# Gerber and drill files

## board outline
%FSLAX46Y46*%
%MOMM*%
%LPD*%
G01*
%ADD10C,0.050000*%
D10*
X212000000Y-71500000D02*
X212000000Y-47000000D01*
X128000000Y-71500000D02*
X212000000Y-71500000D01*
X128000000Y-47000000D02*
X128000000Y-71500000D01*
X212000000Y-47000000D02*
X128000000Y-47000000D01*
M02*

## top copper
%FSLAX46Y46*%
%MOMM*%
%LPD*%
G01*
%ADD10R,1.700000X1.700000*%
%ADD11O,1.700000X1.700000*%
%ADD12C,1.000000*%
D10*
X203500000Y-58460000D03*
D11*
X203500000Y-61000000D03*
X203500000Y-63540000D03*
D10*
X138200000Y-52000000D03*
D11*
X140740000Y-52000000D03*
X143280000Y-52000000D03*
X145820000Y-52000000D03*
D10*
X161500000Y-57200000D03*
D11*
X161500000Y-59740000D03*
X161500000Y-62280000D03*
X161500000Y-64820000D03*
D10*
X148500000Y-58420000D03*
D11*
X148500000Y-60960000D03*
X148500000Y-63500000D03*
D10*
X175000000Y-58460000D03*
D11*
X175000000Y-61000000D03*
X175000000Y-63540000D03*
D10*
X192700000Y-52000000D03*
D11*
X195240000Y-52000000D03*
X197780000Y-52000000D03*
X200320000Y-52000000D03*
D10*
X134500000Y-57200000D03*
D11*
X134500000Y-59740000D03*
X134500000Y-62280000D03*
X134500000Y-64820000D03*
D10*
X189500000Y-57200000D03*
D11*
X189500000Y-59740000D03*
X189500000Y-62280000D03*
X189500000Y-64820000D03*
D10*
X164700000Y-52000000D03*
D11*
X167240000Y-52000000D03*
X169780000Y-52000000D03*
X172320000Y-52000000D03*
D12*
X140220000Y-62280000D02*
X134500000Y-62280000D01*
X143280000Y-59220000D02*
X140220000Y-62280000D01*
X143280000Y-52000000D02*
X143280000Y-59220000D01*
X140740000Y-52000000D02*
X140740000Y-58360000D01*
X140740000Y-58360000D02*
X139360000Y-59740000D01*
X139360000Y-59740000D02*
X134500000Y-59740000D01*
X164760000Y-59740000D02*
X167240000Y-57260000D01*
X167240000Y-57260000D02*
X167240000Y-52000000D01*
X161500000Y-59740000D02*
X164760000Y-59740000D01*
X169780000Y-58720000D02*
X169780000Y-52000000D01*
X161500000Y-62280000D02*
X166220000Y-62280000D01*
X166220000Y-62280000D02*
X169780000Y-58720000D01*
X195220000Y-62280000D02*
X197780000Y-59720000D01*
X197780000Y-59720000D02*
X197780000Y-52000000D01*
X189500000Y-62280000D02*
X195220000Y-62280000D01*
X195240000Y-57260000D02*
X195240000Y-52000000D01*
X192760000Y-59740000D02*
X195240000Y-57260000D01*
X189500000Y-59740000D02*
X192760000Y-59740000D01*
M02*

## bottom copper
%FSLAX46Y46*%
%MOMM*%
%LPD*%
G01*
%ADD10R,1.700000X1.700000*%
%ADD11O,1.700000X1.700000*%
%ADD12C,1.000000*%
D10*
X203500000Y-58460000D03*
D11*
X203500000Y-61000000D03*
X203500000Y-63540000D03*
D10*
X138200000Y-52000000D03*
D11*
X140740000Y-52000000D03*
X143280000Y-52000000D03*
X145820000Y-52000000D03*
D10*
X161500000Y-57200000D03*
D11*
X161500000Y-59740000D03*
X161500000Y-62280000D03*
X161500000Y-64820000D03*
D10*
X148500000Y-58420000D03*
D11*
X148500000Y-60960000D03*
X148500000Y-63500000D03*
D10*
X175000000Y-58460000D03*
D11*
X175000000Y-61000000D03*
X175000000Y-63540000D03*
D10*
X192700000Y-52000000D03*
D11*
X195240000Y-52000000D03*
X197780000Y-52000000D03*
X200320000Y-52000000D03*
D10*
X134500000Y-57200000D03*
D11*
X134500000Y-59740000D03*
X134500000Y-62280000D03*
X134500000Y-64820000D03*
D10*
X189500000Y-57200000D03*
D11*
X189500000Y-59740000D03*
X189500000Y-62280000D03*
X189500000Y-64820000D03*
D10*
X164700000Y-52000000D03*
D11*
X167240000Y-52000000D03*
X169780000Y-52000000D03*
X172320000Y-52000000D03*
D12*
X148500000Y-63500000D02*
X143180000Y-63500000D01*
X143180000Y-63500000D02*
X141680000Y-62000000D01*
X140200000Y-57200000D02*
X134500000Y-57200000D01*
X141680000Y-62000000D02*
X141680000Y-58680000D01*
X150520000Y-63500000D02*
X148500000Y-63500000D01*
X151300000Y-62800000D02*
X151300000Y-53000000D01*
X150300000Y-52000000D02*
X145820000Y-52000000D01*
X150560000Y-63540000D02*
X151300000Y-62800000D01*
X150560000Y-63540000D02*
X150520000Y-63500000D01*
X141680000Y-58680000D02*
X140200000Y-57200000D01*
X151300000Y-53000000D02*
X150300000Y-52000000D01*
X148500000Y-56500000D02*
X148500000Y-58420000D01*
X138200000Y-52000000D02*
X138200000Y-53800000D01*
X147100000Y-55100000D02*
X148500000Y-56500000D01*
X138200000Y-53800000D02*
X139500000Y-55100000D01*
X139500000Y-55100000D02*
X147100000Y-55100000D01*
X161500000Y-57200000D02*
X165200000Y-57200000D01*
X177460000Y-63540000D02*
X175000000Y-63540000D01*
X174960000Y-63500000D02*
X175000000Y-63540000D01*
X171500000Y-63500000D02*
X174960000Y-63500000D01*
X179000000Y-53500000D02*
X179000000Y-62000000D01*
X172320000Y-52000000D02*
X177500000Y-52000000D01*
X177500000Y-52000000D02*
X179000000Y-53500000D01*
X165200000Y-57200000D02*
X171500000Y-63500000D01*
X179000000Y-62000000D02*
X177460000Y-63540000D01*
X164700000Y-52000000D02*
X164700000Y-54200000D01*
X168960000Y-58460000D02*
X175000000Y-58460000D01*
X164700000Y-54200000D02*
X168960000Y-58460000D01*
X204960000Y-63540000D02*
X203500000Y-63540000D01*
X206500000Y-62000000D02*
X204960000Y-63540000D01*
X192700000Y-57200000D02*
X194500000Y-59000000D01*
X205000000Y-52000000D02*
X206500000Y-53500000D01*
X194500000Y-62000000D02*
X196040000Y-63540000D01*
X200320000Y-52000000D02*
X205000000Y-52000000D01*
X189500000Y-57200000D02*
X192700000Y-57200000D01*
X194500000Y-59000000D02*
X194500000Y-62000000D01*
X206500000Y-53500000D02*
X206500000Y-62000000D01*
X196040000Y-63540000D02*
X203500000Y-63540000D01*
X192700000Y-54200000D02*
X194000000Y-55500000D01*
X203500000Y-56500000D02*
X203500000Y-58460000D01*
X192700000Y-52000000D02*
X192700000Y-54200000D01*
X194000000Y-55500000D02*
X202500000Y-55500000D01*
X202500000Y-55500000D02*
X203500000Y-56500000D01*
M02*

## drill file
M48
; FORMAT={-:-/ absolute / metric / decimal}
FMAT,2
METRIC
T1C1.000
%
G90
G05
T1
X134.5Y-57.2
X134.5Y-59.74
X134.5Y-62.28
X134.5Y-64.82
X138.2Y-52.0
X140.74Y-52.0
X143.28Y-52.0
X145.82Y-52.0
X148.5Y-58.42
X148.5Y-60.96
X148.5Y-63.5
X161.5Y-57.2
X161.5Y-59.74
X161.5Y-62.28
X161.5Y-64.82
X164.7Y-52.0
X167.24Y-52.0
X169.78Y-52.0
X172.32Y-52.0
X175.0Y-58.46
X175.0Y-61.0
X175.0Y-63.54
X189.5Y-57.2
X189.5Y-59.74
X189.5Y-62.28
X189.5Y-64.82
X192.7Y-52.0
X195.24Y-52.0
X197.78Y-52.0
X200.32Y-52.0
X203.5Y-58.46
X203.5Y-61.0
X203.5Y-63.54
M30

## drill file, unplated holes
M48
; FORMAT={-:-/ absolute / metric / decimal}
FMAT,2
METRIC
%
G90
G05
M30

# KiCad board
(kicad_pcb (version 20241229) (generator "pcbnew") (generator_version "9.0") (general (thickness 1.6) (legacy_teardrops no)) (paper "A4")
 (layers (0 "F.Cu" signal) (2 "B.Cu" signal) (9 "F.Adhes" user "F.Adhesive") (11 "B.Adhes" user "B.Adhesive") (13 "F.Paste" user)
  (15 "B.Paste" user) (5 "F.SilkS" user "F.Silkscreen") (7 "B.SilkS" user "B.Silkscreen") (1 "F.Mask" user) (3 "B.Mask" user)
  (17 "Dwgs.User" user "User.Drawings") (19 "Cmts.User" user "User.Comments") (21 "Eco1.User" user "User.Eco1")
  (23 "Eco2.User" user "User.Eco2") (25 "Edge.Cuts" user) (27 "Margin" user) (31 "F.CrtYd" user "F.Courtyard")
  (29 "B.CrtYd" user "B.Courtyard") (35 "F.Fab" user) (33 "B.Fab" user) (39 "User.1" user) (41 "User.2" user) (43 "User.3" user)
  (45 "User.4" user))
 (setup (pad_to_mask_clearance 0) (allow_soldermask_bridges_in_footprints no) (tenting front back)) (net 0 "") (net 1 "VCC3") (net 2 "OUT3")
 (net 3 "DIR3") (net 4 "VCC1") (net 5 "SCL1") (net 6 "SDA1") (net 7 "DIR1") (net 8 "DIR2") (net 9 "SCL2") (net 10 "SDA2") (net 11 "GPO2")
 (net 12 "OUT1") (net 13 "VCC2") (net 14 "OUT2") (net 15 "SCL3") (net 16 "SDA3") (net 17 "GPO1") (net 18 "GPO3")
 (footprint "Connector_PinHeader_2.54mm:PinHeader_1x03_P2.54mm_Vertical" (layer "F.Cu") (at 203.5 58.46)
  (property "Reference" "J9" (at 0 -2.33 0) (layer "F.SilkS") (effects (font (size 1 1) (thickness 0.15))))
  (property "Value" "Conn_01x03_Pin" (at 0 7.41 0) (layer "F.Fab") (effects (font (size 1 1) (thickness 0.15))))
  (pad "1" thru_hole rect (at 0 0) (size 1.7 1.7) (drill 1) (layers "*.Cu" "*.Mask") (remove_unused_layers no) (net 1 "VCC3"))
  (pad "2" thru_hole oval (at 0 2.54) (size 1.7 1.7) (drill 1) (layers "*.Cu" "*.Mask") (remove_unused_layers no) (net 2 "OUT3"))
  (pad "3" thru_hole oval (at 0 5.08) (size 1.7 1.7) (drill 1) (layers "*.Cu" "*.Mask") (remove_unused_layers no) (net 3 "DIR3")))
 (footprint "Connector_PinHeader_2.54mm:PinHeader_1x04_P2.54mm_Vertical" (layer "F.Cu") (at 138.2 52 90)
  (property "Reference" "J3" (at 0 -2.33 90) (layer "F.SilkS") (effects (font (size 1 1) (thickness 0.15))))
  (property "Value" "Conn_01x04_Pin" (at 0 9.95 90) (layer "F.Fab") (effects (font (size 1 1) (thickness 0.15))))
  (pad "1" thru_hole rect (at 0 0 90) (size 1.7 1.7) (drill 1) (layers "*.Cu" "*.Mask") (remove_unused_layers no) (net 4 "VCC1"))
  (pad "2" thru_hole oval (at 0 2.54 90) (size 1.7 1.7) (drill 1) (layers "*.Cu" "*.Mask") (remove_unused_layers no) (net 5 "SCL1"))
  (pad "3" thru_hole oval (at 0 5.08 90) (size 1.7 1.7) (drill 1) (layers "*.Cu" "*.Mask") (remove_unused_layers no) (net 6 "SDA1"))
  (pad "4" thru_hole oval (at 0 7.62 90) (size 1.7 1.7) (drill 1) (layers "*.Cu" "*.Mask") (remove_unused_layers no) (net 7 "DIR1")))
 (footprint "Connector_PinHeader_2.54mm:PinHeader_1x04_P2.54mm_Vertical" (layer "F.Cu") (at 161.5 57.2)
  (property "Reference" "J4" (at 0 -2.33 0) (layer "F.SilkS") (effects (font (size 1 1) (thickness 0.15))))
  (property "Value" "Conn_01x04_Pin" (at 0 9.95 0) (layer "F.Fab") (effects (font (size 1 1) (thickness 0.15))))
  (pad "1" thru_hole rect (at 0 0) (size 1.7 1.7) (drill 1) (layers "*.Cu" "*.Mask") (remove_unused_layers no) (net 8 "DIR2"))
  (pad "2" thru_hole oval (at 0 2.54) (size 1.7 1.7) (drill 1) (layers "*.Cu" "*.Mask") (remove_unused_layers no) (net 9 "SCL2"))
  (pad "3" thru_hole oval (at 0 5.08) (size 1.7 1.7) (drill 1) (layers "*.Cu" "*.Mask") (remove_unused_layers no) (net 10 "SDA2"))
  (pad "4" thru_hole oval (at 0 7.62) (size 1.7 1.7) (drill 1) (layers "*.Cu" "*.Mask") (remove_unused_layers no) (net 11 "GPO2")))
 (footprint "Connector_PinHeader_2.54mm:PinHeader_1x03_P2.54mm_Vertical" (layer "F.Cu") (at 148.5 58.42)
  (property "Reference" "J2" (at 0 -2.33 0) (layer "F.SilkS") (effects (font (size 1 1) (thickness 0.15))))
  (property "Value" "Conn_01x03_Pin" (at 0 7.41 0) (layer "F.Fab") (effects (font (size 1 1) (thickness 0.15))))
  (pad "1" thru_hole rect (at 0 0) (size 1.7 1.7) (drill 1) (layers "*.Cu" "*.Mask") (remove_unused_layers no) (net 4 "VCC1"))
  (pad "2" thru_hole oval (at 0 2.54) (size 1.7 1.7) (drill 1) (layers "*.Cu" "*.Mask") (remove_unused_layers no) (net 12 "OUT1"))
  (pad "3" thru_hole oval (at 0 5.08) (size 1.7 1.7) (drill 1) (layers "*.Cu" "*.Mask") (remove_unused_layers no) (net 7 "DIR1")))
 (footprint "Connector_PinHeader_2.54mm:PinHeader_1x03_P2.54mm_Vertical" (layer "F.Cu") (at 175 58.46)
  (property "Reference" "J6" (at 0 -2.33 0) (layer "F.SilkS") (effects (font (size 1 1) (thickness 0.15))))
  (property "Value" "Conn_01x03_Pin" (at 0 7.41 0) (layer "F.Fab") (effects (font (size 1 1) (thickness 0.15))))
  (pad "1" thru_hole rect (at 0 0) (size 1.7 1.7) (drill 1) (layers "*.Cu" "*.Mask") (remove_unused_layers no) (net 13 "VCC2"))
  (pad "2" thru_hole oval (at 0 2.54) (size 1.7 1.7) (drill 1) (layers "*.Cu" "*.Mask") (remove_unused_layers no) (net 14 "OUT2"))
  (pad "3" thru_hole oval (at 0 5.08) (size 1.7 1.7) (drill 1) (layers "*.Cu" "*.Mask") (remove_unused_layers no) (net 8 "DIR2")))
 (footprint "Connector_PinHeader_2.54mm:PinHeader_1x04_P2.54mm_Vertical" (layer "F.Cu") (at 192.7 52 90)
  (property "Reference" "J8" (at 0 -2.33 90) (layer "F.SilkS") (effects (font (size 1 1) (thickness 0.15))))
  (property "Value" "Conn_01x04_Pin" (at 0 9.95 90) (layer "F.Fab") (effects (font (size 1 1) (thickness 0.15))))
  (pad "1" thru_hole rect (at 0 0 90) (size 1.7 1.7) (drill 1) (layers "*.Cu" "*.Mask") (remove_unused_layers no) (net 1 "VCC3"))
  (pad "2" thru_hole oval (at 0 2.54 90) (size 1.7 1.7) (drill 1) (layers "*.Cu" "*.Mask") (remove_unused_layers no) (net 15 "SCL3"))
  (pad "3" thru_hole oval (at 0 5.08 90) (size 1.7 1.7) (drill 1) (layers "*.Cu" "*.Mask") (remove_unused_layers no) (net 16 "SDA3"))
  (pad "4" thru_hole oval (at 0 7.62 90) (size 1.7 1.7) (drill 1) (layers "*.Cu" "*.Mask") (remove_unused_layers no) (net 3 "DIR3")))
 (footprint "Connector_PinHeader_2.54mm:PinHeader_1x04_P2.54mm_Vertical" (layer "F.Cu") (at 134.5 57.2)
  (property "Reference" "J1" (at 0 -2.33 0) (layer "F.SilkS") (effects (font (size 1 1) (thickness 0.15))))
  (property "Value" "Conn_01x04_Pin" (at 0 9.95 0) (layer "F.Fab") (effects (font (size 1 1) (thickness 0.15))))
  (pad "1" thru_hole rect (at 0 0) (size 1.7 1.7) (drill 1) (layers "*.Cu" "*.Mask") (remove_unused_layers no) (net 7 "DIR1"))
  (pad "2" thru_hole oval (at 0 2.54) (size 1.7 1.7) (drill 1) (layers "*.Cu" "*.Mask") (remove_unused_layers no) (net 5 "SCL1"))
  (pad "3" thru_hole oval (at 0 5.08) (size 1.7 1.7) (drill 1) (layers "*.Cu" "*.Mask") (remove_unused_layers no) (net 6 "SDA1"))
  (pad "4" thru_hole oval (at 0 7.62) (size 1.7 1.7) (drill 1) (layers "*.Cu" "*.Mask") (remove_unused_layers no) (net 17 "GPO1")))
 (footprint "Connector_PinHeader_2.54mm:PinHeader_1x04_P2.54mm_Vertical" (layer "F.Cu") (at 189.5 57.2)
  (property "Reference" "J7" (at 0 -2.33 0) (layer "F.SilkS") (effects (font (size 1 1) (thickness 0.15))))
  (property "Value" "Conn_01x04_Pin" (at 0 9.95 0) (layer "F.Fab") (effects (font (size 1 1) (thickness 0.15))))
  (pad "1" thru_hole rect (at 0 0) (size 1.7 1.7) (drill 1) (layers "*.Cu" "*.Mask") (remove_unused_layers no) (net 3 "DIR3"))
  (pad "2" thru_hole oval (at 0 2.54) (size 1.7 1.7) (drill 1) (layers "*.Cu" "*.Mask") (remove_unused_layers no) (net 15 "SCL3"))
  (pad "3" thru_hole oval (at 0 5.08) (size 1.7 1.7) (drill 1) (layers "*.Cu" "*.Mask") (remove_unused_layers no) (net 16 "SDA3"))
  (pad "4" thru_hole oval (at 0 7.62) (size 1.7 1.7) (drill 1) (layers "*.Cu" "*.Mask") (remove_unused_layers no) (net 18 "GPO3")))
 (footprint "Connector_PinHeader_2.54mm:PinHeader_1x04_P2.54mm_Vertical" (layer "F.Cu") (at 164.7 52 90)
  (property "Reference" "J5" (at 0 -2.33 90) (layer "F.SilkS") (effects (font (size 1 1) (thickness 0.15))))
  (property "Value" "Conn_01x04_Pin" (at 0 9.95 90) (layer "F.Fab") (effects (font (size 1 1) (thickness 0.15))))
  (pad "1" thru_hole rect (at 0 0 90) (size 1.7 1.7) (drill 1) (layers "*.Cu" "*.Mask") (remove_unused_layers no) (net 13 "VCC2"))
  (pad "2" thru_hole oval (at 0 2.54 90) (size 1.7 1.7) (drill 1) (layers "*.Cu" "*.Mask") (remove_unused_layers no) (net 9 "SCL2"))
  (pad "3" thru_hole oval (at 0 5.08 90) (size 1.7 1.7) (drill 1) (layers "*.Cu" "*.Mask") (remove_unused_layers no) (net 10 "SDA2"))
  (pad "4" thru_hole oval (at 0 7.62 90) (size 1.7 1.7) (drill 1) (layers "*.Cu" "*.Mask") (remove_unused_layers no) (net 8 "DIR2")))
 (gr_line (start 212 71.5) (end 212 47) (stroke (width 0.05) (type default)) (layer "Edge.Cuts"))
 (gr_line (start 128 71.5) (end 212 71.5) (stroke (width 0.05) (type default)) (layer "Edge.Cuts"))
 (gr_line (start 128 47) (end 128 71.5) (stroke (width 0.05) (type default)) (layer "Edge.Cuts"))
 (gr_line (start 212 47) (end 128 47) (stroke (width 0.05) (type default)) (layer "Edge.Cuts"))
 (segment (start 148.5 63.5) (end 143.18 63.5) (width 1) (layer "B.Cu") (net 7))
 (segment (start 143.18 63.5) (end 141.68 62) (width 1) (layer "B.Cu") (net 7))
 (segment (start 140.2 57.2) (end 134.5 57.2) (width 1) (layer "B.Cu") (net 7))
 (segment (start 141.68 62) (end 141.68 58.68) (width 1) (layer "B.Cu") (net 7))
 (segment (start 150.52 63.5) (end 148.5 63.5) (width 1) (layer "B.Cu") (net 7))
 (segment (start 151.3 62.8) (end 151.3 53) (width 1) (layer "B.Cu") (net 7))
 (segment (start 150.3 52) (end 145.82 52) (width 1) (layer "B.Cu") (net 7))
 (segment (start 150.56 63.54) (end 151.3 62.8) (width 1) (layer "B.Cu") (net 7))
 (segment (start 150.56 63.54) (end 150.52 63.5) (width 1) (layer "B.Cu") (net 7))
 (segment (start 141.68 58.68) (end 140.2 57.2) (width 1) (layer "B.Cu") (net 7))
 (segment (start 151.3 53) (end 150.3 52) (width 1) (layer "B.Cu") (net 7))
 (segment (start 140.22 62.28) (end 134.5 62.28) (width 1) (layer "F.Cu") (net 6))
 (segment (start 143.28 59.22) (end 140.22 62.28) (width 1) (layer "F.Cu") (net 6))
 (segment (start 143.28 52) (end 143.28 59.22) (width 1) (layer "F.Cu") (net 6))
 (segment (start 140.74 52) (end 140.74 58.36) (width 1) (layer "F.Cu") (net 5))
 (segment (start 140.74 58.36) (end 139.36 59.74) (width 1) (layer "F.Cu") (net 5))
 (segment (start 139.36 59.74) (end 134.5 59.74) (width 1) (layer "F.Cu") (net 5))
 (segment (start 148.5 56.5) (end 148.5 58.42) (width 1) (layer "B.Cu") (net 4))
 (segment (start 138.2 52) (end 138.2 53.8) (width 1) (layer "B.Cu") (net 4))
 (segment (start 147.1 55.1) (end 148.5 56.5) (width 1) (layer "B.Cu") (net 4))
 (segment (start 138.2 53.8) (end 139.5 55.1) (width 1) (layer "B.Cu") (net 4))
 (segment (start 139.5 55.1) (end 147.1 55.1) (width 1) (layer "B.Cu") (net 4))
 (segment (start 164.76 59.74) (end 167.24 57.26) (width 1) (layer "F.Cu") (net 9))
 (segment (start 167.24 57.26) (end 167.24 52) (width 1) (layer "F.Cu") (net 9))
 (segment (start 161.5 59.74) (end 164.76 59.74) (width 1) (layer "F.Cu") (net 9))
 (segment (start 161.5 57.2) (end 165.2 57.2) (width 1) (layer "B.Cu") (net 8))
 (segment (start 177.46 63.54) (end 175 63.54) (width 1) (layer "B.Cu") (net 8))
 (segment (start 174.96 63.5) (end 175 63.54) (width 1) (layer "B.Cu") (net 8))
 (segment (start 171.5 63.5) (end 174.96 63.5) (width 1) (layer "B.Cu") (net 8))
 (segment (start 179 53.5) (end 179 62) (width 1) (layer "B.Cu") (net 8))
 (segment (start 172.32 52) (end 177.5 52) (width 1) (layer "B.Cu") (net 8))
 (segment (start 177.5 52) (end 179 53.5) (width 1) (layer "B.Cu") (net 8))
 (segment (start 165.2 57.2) (end 171.5 63.5) (width 1) (layer "B.Cu") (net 8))
 (segment (start 179 62) (end 177.46 63.54) (width 1) (layer "B.Cu") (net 8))
 (segment (start 169.78 58.72) (end 169.78 52) (width 1) (layer "F.Cu") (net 10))
 (segment (start 161.5 62.28) (end 166.22 62.28) (width 1) (layer "F.Cu") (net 10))
 (segment (start 166.22 62.28) (end 169.78 58.72) (width 1) (layer "F.Cu") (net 10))
 (segment (start 164.7 52) (end 164.7 54.2) (width 1) (layer "B.Cu") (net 13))
 (segment (start 168.96 58.46) (end 175 58.46) (width 1) (layer "B.Cu") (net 13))
 (segment (start 164.7 54.2) (end 168.96 58.46) (width 1) (layer "B.Cu") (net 13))
 (segment (start 195.22 62.28) (end 197.78 59.72) (width 1) (layer "F.Cu") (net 16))
 (segment (start 197.78 59.72) (end 197.78 52) (width 1) (layer "F.Cu") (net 16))
 (segment (start 189.5 62.28) (end 195.22 62.28) (width 1) (layer "F.Cu") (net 16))
 (segment (start 195.24 57.26) (end 195.24 52) (width 1) (layer "F.Cu") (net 15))
 (segment (start 192.76 59.74) (end 195.24 57.26) (width 1) (layer "F.Cu") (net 15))
 (segment (start 189.5 59.74) (end 192.76 59.74) (width 1) (layer "F.Cu") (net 15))
 (segment (start 204.96 63.54) (end 203.5 63.54) (width 1) (layer "B.Cu") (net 3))
 (segment (start 206.5 62) (end 204.96 63.54) (width 1) (layer "B.Cu") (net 3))
 (segment (start 192.7 57.2) (end 194.5 59) (width 1) (layer "B.Cu") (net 3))
 (segment (start 205 52) (end 206.5 53.5) (width 1) (layer "B.Cu") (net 3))
 (segment (start 194.5 62) (end 196.04 63.54) (width 1) (layer "B.Cu") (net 3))
 (segment (start 200.32 52) (end 205 52) (width 1) (layer "B.Cu") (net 3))
 (segment (start 189.5 57.2) (end 192.7 57.2) (width 1) (layer "B.Cu") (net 3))
 (segment (start 194.5 59) (end 194.5 62) (width 1) (layer "B.Cu") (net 3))
 (segment (start 206.5 53.5) (end 206.5 62) (width 1) (layer "B.Cu") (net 3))
 (segment (start 196.04 63.54) (end 203.5 63.54) (width 1) (layer "B.Cu") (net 3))
 (segment (start 192.7 54.2) (end 194 55.5) (width 1) (layer "B.Cu") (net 1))
 (segment (start 203.5 56.5) (end 203.5 58.46) (width 1) (layer "B.Cu") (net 1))
 (segment (start 192.7 52) (end 192.7 54.2) (width 1) (layer "B.Cu") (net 1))
 (segment (start 194 55.5) (end 202.5 55.5) (width 1) (layer "B.Cu") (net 1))
 (segment (start 202.5 55.5) (end 203.5 56.5) (width 1) (layer "B.Cu") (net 1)))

